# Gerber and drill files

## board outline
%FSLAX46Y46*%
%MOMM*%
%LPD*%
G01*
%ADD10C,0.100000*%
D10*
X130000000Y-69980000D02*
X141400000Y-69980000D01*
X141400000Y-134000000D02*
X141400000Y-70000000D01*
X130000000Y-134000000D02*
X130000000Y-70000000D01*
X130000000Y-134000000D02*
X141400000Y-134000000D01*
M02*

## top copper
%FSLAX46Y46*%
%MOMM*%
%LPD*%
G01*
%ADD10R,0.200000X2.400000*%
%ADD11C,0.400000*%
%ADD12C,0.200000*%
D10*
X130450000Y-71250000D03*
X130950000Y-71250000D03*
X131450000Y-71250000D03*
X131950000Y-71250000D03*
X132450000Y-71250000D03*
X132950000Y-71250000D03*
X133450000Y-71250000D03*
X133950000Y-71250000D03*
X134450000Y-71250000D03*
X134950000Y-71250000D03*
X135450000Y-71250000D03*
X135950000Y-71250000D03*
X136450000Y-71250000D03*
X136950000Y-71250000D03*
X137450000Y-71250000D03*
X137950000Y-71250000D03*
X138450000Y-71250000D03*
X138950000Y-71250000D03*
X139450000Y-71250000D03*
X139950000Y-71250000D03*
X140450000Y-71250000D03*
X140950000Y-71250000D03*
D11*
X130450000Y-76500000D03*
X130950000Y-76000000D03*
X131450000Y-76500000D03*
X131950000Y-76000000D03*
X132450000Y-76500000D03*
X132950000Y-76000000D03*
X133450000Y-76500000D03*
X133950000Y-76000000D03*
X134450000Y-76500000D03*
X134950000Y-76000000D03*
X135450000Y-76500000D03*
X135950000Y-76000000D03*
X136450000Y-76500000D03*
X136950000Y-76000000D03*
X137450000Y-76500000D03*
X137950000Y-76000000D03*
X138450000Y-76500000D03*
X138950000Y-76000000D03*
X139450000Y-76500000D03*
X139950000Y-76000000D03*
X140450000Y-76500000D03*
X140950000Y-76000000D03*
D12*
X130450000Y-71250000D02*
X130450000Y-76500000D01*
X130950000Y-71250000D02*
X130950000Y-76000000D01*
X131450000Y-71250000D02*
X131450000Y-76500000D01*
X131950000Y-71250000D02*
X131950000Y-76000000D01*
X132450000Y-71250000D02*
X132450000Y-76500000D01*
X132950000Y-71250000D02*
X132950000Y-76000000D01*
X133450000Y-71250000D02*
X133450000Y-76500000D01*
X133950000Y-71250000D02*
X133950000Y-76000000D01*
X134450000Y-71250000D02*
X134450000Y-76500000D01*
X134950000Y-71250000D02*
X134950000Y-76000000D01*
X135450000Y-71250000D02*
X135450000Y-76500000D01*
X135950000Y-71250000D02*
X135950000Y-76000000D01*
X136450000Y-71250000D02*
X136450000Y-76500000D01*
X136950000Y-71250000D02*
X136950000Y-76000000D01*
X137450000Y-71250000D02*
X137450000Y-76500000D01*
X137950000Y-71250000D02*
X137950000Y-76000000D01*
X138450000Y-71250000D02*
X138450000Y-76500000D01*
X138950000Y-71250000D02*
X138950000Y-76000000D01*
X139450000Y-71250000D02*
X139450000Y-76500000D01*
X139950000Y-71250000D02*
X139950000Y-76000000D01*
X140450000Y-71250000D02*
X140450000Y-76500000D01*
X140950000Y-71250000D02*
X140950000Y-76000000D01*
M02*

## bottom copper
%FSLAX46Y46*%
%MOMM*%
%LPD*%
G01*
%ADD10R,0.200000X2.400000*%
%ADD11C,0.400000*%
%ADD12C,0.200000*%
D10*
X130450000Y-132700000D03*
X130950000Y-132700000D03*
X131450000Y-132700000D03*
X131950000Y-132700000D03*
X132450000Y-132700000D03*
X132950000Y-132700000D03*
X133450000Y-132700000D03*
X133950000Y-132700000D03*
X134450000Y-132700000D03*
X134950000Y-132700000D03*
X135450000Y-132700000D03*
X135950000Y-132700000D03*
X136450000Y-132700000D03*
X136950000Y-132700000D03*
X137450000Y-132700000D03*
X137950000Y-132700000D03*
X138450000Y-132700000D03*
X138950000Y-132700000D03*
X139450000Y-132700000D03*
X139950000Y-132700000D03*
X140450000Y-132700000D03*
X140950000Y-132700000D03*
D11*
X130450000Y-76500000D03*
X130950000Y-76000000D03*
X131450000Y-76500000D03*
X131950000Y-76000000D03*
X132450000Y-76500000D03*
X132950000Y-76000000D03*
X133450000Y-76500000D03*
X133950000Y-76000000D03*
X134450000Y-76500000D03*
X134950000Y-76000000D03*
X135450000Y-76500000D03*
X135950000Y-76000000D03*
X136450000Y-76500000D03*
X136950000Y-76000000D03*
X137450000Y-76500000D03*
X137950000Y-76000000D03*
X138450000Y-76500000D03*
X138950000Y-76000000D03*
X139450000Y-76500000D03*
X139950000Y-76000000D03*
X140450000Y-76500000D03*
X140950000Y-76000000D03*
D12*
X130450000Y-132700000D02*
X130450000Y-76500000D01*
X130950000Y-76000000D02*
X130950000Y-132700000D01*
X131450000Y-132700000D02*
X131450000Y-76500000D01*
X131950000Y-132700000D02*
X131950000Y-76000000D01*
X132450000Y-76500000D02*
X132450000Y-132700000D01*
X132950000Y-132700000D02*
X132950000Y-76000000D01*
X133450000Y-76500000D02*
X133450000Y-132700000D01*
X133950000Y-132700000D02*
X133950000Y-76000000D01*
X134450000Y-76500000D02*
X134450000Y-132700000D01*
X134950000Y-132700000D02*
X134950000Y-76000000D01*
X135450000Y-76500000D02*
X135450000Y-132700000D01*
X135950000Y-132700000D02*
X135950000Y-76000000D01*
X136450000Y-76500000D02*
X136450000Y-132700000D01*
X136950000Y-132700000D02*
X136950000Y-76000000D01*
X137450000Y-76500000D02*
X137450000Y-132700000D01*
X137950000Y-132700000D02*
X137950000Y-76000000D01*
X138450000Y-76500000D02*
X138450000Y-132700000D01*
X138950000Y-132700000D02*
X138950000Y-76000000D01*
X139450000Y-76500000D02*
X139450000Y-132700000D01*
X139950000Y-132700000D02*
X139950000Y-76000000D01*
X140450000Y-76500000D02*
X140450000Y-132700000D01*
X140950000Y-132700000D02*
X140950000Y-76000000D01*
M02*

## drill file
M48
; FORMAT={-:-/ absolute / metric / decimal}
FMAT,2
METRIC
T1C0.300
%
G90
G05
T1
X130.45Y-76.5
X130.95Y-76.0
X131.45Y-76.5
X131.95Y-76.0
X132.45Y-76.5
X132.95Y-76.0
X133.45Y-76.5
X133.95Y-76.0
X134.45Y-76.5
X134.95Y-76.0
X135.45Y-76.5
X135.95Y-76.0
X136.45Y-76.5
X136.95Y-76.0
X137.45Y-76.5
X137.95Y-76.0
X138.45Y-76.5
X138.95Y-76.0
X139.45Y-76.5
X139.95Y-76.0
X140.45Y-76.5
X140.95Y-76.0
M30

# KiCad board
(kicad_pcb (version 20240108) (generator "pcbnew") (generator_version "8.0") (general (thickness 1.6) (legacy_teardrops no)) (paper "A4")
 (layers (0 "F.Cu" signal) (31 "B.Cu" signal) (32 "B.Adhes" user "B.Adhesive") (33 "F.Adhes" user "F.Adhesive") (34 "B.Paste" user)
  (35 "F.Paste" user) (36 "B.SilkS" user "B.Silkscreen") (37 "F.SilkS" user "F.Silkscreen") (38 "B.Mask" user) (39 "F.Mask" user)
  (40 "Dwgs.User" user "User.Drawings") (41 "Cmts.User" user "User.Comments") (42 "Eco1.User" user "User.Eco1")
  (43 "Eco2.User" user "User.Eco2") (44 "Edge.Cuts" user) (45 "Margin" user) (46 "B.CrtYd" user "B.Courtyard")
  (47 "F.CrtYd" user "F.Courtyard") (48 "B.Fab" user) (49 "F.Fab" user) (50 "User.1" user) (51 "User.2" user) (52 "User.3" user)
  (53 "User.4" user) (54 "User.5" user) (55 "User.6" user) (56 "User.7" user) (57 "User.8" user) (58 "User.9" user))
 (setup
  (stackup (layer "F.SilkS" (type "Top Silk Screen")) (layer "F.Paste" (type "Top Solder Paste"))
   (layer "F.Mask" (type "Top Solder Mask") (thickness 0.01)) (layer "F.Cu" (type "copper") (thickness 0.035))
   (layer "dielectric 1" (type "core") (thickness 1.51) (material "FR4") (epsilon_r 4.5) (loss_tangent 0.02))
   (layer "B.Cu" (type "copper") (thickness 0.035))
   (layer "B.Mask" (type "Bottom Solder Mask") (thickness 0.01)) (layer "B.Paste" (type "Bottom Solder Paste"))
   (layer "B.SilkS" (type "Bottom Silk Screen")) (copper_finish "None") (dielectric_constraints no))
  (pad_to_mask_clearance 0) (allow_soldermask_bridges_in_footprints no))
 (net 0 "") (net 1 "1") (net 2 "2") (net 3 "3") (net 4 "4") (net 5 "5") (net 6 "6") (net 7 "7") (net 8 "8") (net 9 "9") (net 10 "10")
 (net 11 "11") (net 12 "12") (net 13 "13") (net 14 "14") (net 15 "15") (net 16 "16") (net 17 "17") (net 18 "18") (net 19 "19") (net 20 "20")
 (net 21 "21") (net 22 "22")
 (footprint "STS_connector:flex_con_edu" (layer "F.Cu") (at 130 74.6)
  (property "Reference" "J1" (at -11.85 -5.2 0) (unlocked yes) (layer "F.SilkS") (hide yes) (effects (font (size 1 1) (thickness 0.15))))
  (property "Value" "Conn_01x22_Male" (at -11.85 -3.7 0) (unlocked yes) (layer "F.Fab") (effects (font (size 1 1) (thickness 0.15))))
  (pad "1" smd rect (at 0.45 -3.35) (size 0.2 2.4) (layers "F.Cu" "F.Paste" "F.Mask") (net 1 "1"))
  (pad "2" smd rect (at 0.95 -3.35) (size 0.2 2.4) (layers "F.Cu" "F.Paste" "F.Mask") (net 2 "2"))
  (pad "3" smd rect (at 1.45 -3.35) (size 0.2 2.4) (layers "F.Cu" "F.Paste" "F.Mask") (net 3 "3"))
  (pad "4" smd rect (at 1.95 -3.35) (size 0.2 2.4) (layers "F.Cu" "F.Paste" "F.Mask") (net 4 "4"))
  (pad "5" smd rect (at 2.45 -3.35) (size 0.2 2.4) (layers "F.Cu" "F.Paste" "F.Mask") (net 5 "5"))
  (pad "6" smd rect (at 2.95 -3.35) (size 0.2 2.4) (layers "F.Cu" "F.Paste" "F.Mask") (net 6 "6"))
  (pad "7" smd rect (at 3.45 -3.35) (size 0.2 2.4) (layers "F.Cu" "F.Paste" "F.Mask") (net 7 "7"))
  (pad "8" smd rect (at 3.95 -3.35) (size 0.2 2.4) (layers "F.Cu" "F.Paste" "F.Mask") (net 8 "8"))
  (pad "9" smd rect (at 4.45 -3.35) (size 0.2 2.4) (layers "F.Cu" "F.Paste" "F.Mask") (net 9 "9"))
  (pad "10" smd rect (at 4.95 -3.35) (size 0.2 2.4) (layers "F.Cu" "F.Paste" "F.Mask") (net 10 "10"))
  (pad "11" smd rect (at 5.45 -3.35) (size 0.2 2.4) (layers "F.Cu" "F.Paste" "F.Mask") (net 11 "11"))
  (pad "12" smd rect (at 5.95 -3.35) (size 0.2 2.4) (layers "F.Cu" "F.Paste" "F.Mask") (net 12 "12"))
  (pad "13" smd rect (at 6.45 -3.35) (size 0.2 2.4) (layers "F.Cu" "F.Paste" "F.Mask") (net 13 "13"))
  (pad "14" smd rect (at 6.95 -3.35) (size 0.2 2.4) (layers "F.Cu" "F.Paste" "F.Mask") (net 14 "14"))
  (pad "15" smd rect (at 7.45 -3.35) (size 0.2 2.4) (layers "F.Cu" "F.Paste" "F.Mask") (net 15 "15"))
  (pad "16" smd rect (at 7.95 -3.35) (size 0.2 2.4) (layers "F.Cu" "F.Paste" "F.Mask") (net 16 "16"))
  (pad "17" smd rect (at 8.45 -3.35) (size 0.2 2.4) (layers "F.Cu" "F.Paste" "F.Mask") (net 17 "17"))
  (pad "18" smd rect (at 8.95 -3.35) (size 0.2 2.4) (layers "F.Cu" "F.Paste" "F.Mask") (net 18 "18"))
  (pad "19" smd rect (at 9.45 -3.35) (size 0.2 2.4) (layers "F.Cu" "F.Paste" "F.Mask") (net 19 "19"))
  (pad "20" smd rect (at 9.95 -3.35) (size 0.2 2.4) (layers "F.Cu" "F.Paste" "F.Mask") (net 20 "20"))
  (pad "21" smd rect (at 10.45 -3.35) (size 0.2 2.4) (layers "F.Cu" "F.Paste" "F.Mask") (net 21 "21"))
  (pad "22" smd rect (at 10.95 -3.35) (size 0.2 2.4) (layers "F.Cu" "F.Paste" "F.Mask") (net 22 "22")))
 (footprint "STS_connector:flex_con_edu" (layer "B.Cu") (at 130 129.35)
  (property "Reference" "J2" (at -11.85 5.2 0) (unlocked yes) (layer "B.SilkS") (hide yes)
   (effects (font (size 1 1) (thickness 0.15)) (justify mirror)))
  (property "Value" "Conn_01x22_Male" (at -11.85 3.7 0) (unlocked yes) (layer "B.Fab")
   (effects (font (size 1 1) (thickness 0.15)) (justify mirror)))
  (pad "1" smd rect (at 0.45 3.35) (size 0.2 2.4) (layers "B.Cu" "B.Paste" "B.Mask") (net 1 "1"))
  (pad "2" smd rect (at 0.95 3.35) (size 0.2 2.4) (layers "B.Cu" "B.Paste" "B.Mask") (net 2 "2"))
  (pad "3" smd rect (at 1.45 3.35) (size 0.2 2.4) (layers "B.Cu" "B.Paste" "B.Mask") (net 3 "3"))
  (pad "4" smd rect (at 1.95 3.35) (size 0.2 2.4) (layers "B.Cu" "B.Paste" "B.Mask") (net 4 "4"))
  (pad "5" smd rect (at 2.45 3.35) (size 0.2 2.4) (layers "B.Cu" "B.Paste" "B.Mask") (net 5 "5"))
  (pad "6" smd rect (at 2.95 3.35) (size 0.2 2.4) (layers "B.Cu" "B.Paste" "B.Mask") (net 6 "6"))
  (pad "7" smd rect (at 3.45 3.35) (size 0.2 2.4) (layers "B.Cu" "B.Paste" "B.Mask") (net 7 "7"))
  (pad "8" smd rect (at 3.95 3.35) (size 0.2 2.4) (layers "B.Cu" "B.Paste" "B.Mask") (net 8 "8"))
  (pad "9" smd rect (at 4.45 3.35) (size 0.2 2.4) (layers "B.Cu" "B.Paste" "B.Mask") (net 9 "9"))
  (pad "10" smd rect (at 4.95 3.35) (size 0.2 2.4) (layers "B.Cu" "B.Paste" "B.Mask") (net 10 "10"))
  (pad "11" smd rect (at 5.45 3.35) (size 0.2 2.4) (layers "B.Cu" "B.Paste" "B.Mask") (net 11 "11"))
  (pad "12" smd rect (at 5.95 3.35) (size 0.2 2.4) (layers "B.Cu" "B.Paste" "B.Mask") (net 12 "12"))
  (pad "13" smd rect (at 6.45 3.35) (size 0.2 2.4) (layers "B.Cu" "B.Paste" "B.Mask") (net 13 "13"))
  (pad "14" smd rect (at 6.95 3.35) (size 0.2 2.4) (layers "B.Cu" "B.Paste" "B.Mask") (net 14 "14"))
  (pad "15" smd rect (at 7.45 3.35) (size 0.2 2.4) (layers "B.Cu" "B.Paste" "B.Mask") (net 15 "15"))
  (pad "16" smd rect (at 7.95 3.35) (size 0.2 2.4) (layers "B.Cu" "B.Paste" "B.Mask") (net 16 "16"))
  (pad "17" smd rect (at 8.45 3.35) (size 0.2 2.4) (layers "B.Cu" "B.Paste" "B.Mask") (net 17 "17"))
  (pad "18" smd rect (at 8.95 3.35) (size 0.2 2.4) (layers "B.Cu" "B.Paste" "B.Mask") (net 18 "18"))
  (pad "19" smd rect (at 9.45 3.35) (size 0.2 2.4) (layers "B.Cu" "B.Paste" "B.Mask") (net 19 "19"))
  (pad "20" smd rect (at 9.95 3.35) (size 0.2 2.4) (layers "B.Cu" "B.Paste" "B.Mask") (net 20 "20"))
  (pad "21" smd rect (at 10.45 3.35) (size 0.2 2.4) (layers "B.Cu" "B.Paste" "B.Mask") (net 21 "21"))
  (pad "22" smd rect (at 10.95 3.35) (size 0.2 2.4) (layers "B.Cu" "B.Paste" "B.Mask") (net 22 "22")))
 (gr_line (start 130 69.98) (end 141.4 69.98) (stroke (width 0.1) (type solid)) (layer "Edge.Cuts"))
 (gr_line (start 141.4 134) (end 141.4 70) (stroke (width 0.1) (type solid)) (layer "Edge.Cuts"))
 (gr_line (start 130 134) (end 130 70) (stroke (width 0.1) (type solid)) (layer "Edge.Cuts"))
 (gr_line (start 130 134) (end 141.4 134) (stroke (width 0.1) (type solid)) (layer "Edge.Cuts"))
 (segment (start 130.45 71.25) (end 130.45 76.5) (width 0.2) (layer "F.Cu") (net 1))
 (via (at 130.45 76.5) (size 0.4) (drill 0.3) (layers "F.Cu" "B.Cu") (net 1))
 (segment (start 130.45 132.7) (end 130.45 76.5) (width 0.2) (layer "B.Cu") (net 1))
 (segment (start 130.95 71.25) (end 130.95 76) (width 0.2) (layer "F.Cu") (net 2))
 (via (at 130.95 76) (size 0.4) (drill 0.3) (layers "F.Cu" "B.Cu") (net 2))
 (segment (start 130.95 76) (end 130.95 132.7) (width 0.2) (layer "B.Cu") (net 2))
 (segment (start 131.45 71.25) (end 131.45 76.5) (width 0.2) (layer "F.Cu") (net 3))
 (via (at 131.45 76.5) (size 0.4) (drill 0.3) (layers "F.Cu" "B.Cu") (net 3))
 (segment (start 131.45 132.7) (end 131.45 76.5) (width 0.2) (layer "B.Cu") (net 3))
 (segment (start 131.95 71.25) (end 131.95 76) (width 0.2) (layer "F.Cu") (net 4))
 (via (at 131.95 76) (size 0.4) (drill 0.3) (layers "F.Cu" "B.Cu") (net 4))
 (segment (start 131.95 132.7) (end 131.95 76) (width 0.2) (layer "B.Cu") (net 4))
 (segment (start 132.45 71.25) (end 132.45 76.5) (width 0.2) (layer "F.Cu") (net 5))
 (via (at 132.45 76.5) (size 0.4) (drill 0.3) (layers "F.Cu" "B.Cu") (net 5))
 (segment (start 132.45 76.5) (end 132.45 132.7) (width 0.2) (layer "B.Cu") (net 5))
 (segment (start 132.95 71.25) (end 132.95 76) (width 0.2) (layer "F.Cu") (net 6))
 (via (at 132.95 76) (size 0.4) (drill 0.3) (layers "F.Cu" "B.Cu") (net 6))
 (segment (start 132.95 132.7) (end 132.95 76) (width 0.2) (layer "B.Cu") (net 6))
 (segment (start 133.45 71.25) (end 133.45 76.5) (width 0.2) (layer "F.Cu") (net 7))
 (via (at 133.45 76.5) (size 0.4) (drill 0.3) (layers "F.Cu" "B.Cu") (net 7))
 (segment (start 133.45 76.5) (end 133.45 132.7) (width 0.2) (layer "B.Cu") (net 7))
 (segment (start 133.95 71.25) (end 133.95 76) (width 0.2) (layer "F.Cu") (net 8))
 (via (at 133.95 76) (size 0.4) (drill 0.3) (layers "F.Cu" "B.Cu") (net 8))
 (segment (start 133.95 132.7) (end 133.95 76) (width 0.2) (layer "B.Cu") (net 8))
 (segment (start 134.45 71.25) (end 134.45 76.5) (width 0.2) (layer "F.Cu") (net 9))
 (via (at 134.45 76.5) (size 0.4) (drill 0.3) (layers "F.Cu" "B.Cu") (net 9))
 (segment (start 134.45 76.5) (end 134.45 132.7) (width 0.2) (layer "B.Cu") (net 9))
 (segment (start 134.95 71.25) (end 134.95 76) (width 0.2) (layer "F.Cu") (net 10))
 (via (at 134.95 76) (size 0.4) (drill 0.3) (layers "F.Cu" "B.Cu") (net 10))
 (segment (start 134.95 132.7) (end 134.95 76) (width 0.2) (layer "B.Cu") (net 10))
 (segment (start 135.45 71.25) (end 135.45 76.5) (width 0.2) (layer "F.Cu") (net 11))
 (via (at 135.45 76.5) (size 0.4) (drill 0.3) (layers "F.Cu" "B.Cu") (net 11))
 (segment (start 135.45 76.5) (end 135.45 132.7) (width 0.2) (layer "B.Cu") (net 11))
 (segment (start 135.95 71.25) (end 135.95 76) (width 0.2) (layer "F.Cu") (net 12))
 (via (at 135.95 76) (size 0.4) (drill 0.3) (layers "F.Cu" "B.Cu") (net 12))
 (segment (start 135.95 132.7) (end 135.95 76) (width 0.2) (layer "B.Cu") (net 12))
 (segment (start 136.45 71.25) (end 136.45 76.5) (width 0.2) (layer "F.Cu") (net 13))
 (via (at 136.45 76.5) (size 0.4) (drill 0.3) (layers "F.Cu" "B.Cu") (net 13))
 (segment (start 136.45 76.5) (end 136.45 132.7) (width 0.2) (layer "B.Cu") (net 13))
 (segment (start 136.95 71.25) (end 136.95 76) (width 0.2) (layer "F.Cu") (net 14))
 (via (at 136.95 76) (size 0.4) (drill 0.3) (layers "F.Cu" "B.Cu") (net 14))
 (segment (start 136.95 132.7) (end 136.95 76) (width 0.2) (layer "B.Cu") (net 14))
 (segment (start 137.45 71.25) (end 137.45 76.5) (width 0.2) (layer "F.Cu") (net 15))
 (via (at 137.45 76.5) (size 0.4) (drill 0.3) (layers "F.Cu" "B.Cu") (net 15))
 (segment (start 137.45 76.5) (end 137.45 132.7) (width 0.2) (layer "B.Cu") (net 15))
 (segment (start 137.95 71.25) (end 137.95 76) (width 0.2) (layer "F.Cu") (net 16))
 (via (at 137.95 76) (size 0.4) (drill 0.3) (layers "F.Cu" "B.Cu") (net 16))
 (segment (start 137.95 132.7) (end 137.95 76) (width 0.2) (layer "B.Cu") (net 16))
 (segment (start 138.45 71.25) (end 138.45 76.5) (width 0.2) (layer "F.Cu") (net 17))
 (via (at 138.45 76.5) (size 0.4) (drill 0.3) (layers "F.Cu" "B.Cu") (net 17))
 (segment (start 138.45 76.5) (end 138.45 132.7) (width 0.2) (layer "B.Cu") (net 17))
 (segment (start 138.95 71.25) (end 138.95 76) (width 0.2) (layer "F.Cu") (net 18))
 (via (at 138.95 76) (size 0.4) (drill 0.3) (layers "F.Cu" "B.Cu") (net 18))
 (segment (start 138.95 132.7) (end 138.95 76) (width 0.2) (layer "B.Cu") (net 18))
 (segment (start 139.45 71.25) (end 139.45 76.5) (width 0.2) (layer "F.Cu") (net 19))
 (via (at 139.45 76.5) (size 0.4) (drill 0.3) (layers "F.Cu" "B.Cu") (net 19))
 (segment (start 139.45 76.5) (end 139.45 132.7) (width 0.2) (layer "B.Cu") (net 19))
 (segment (start 139.95 71.25) (end 139.95 76) (width 0.2) (layer "F.Cu") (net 20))
 (via (at 139.95 76) (size 0.4) (drill 0.3) (layers "F.Cu" "B.Cu") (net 20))
 (segment (start 139.95 132.7) (end 139.95 76) (width 0.2) (layer "B.Cu") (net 20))
 (segment (start 140.45 71.25) (end 140.45 76.5) (width 0.2) (layer "F.Cu") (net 21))
 (via (at 140.45 76.5) (size 0.4) (drill 0.3) (layers "F.Cu" "B.Cu") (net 21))
 (segment (start 140.45 76.5) (end 140.45 132.7) (width 0.2) (layer "B.Cu") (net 21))
 (segment (start 140.95 71.25) (end 140.95 76) (width 0.2) (layer "F.Cu") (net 22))
 (via (at 140.95 76) (size 0.4) (drill 0.3) (layers "F.Cu" "B.Cu") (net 22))
 (segment (start 140.95 132.7) (end 140.95 76) (width 0.2) (layer "B.Cu") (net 22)))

